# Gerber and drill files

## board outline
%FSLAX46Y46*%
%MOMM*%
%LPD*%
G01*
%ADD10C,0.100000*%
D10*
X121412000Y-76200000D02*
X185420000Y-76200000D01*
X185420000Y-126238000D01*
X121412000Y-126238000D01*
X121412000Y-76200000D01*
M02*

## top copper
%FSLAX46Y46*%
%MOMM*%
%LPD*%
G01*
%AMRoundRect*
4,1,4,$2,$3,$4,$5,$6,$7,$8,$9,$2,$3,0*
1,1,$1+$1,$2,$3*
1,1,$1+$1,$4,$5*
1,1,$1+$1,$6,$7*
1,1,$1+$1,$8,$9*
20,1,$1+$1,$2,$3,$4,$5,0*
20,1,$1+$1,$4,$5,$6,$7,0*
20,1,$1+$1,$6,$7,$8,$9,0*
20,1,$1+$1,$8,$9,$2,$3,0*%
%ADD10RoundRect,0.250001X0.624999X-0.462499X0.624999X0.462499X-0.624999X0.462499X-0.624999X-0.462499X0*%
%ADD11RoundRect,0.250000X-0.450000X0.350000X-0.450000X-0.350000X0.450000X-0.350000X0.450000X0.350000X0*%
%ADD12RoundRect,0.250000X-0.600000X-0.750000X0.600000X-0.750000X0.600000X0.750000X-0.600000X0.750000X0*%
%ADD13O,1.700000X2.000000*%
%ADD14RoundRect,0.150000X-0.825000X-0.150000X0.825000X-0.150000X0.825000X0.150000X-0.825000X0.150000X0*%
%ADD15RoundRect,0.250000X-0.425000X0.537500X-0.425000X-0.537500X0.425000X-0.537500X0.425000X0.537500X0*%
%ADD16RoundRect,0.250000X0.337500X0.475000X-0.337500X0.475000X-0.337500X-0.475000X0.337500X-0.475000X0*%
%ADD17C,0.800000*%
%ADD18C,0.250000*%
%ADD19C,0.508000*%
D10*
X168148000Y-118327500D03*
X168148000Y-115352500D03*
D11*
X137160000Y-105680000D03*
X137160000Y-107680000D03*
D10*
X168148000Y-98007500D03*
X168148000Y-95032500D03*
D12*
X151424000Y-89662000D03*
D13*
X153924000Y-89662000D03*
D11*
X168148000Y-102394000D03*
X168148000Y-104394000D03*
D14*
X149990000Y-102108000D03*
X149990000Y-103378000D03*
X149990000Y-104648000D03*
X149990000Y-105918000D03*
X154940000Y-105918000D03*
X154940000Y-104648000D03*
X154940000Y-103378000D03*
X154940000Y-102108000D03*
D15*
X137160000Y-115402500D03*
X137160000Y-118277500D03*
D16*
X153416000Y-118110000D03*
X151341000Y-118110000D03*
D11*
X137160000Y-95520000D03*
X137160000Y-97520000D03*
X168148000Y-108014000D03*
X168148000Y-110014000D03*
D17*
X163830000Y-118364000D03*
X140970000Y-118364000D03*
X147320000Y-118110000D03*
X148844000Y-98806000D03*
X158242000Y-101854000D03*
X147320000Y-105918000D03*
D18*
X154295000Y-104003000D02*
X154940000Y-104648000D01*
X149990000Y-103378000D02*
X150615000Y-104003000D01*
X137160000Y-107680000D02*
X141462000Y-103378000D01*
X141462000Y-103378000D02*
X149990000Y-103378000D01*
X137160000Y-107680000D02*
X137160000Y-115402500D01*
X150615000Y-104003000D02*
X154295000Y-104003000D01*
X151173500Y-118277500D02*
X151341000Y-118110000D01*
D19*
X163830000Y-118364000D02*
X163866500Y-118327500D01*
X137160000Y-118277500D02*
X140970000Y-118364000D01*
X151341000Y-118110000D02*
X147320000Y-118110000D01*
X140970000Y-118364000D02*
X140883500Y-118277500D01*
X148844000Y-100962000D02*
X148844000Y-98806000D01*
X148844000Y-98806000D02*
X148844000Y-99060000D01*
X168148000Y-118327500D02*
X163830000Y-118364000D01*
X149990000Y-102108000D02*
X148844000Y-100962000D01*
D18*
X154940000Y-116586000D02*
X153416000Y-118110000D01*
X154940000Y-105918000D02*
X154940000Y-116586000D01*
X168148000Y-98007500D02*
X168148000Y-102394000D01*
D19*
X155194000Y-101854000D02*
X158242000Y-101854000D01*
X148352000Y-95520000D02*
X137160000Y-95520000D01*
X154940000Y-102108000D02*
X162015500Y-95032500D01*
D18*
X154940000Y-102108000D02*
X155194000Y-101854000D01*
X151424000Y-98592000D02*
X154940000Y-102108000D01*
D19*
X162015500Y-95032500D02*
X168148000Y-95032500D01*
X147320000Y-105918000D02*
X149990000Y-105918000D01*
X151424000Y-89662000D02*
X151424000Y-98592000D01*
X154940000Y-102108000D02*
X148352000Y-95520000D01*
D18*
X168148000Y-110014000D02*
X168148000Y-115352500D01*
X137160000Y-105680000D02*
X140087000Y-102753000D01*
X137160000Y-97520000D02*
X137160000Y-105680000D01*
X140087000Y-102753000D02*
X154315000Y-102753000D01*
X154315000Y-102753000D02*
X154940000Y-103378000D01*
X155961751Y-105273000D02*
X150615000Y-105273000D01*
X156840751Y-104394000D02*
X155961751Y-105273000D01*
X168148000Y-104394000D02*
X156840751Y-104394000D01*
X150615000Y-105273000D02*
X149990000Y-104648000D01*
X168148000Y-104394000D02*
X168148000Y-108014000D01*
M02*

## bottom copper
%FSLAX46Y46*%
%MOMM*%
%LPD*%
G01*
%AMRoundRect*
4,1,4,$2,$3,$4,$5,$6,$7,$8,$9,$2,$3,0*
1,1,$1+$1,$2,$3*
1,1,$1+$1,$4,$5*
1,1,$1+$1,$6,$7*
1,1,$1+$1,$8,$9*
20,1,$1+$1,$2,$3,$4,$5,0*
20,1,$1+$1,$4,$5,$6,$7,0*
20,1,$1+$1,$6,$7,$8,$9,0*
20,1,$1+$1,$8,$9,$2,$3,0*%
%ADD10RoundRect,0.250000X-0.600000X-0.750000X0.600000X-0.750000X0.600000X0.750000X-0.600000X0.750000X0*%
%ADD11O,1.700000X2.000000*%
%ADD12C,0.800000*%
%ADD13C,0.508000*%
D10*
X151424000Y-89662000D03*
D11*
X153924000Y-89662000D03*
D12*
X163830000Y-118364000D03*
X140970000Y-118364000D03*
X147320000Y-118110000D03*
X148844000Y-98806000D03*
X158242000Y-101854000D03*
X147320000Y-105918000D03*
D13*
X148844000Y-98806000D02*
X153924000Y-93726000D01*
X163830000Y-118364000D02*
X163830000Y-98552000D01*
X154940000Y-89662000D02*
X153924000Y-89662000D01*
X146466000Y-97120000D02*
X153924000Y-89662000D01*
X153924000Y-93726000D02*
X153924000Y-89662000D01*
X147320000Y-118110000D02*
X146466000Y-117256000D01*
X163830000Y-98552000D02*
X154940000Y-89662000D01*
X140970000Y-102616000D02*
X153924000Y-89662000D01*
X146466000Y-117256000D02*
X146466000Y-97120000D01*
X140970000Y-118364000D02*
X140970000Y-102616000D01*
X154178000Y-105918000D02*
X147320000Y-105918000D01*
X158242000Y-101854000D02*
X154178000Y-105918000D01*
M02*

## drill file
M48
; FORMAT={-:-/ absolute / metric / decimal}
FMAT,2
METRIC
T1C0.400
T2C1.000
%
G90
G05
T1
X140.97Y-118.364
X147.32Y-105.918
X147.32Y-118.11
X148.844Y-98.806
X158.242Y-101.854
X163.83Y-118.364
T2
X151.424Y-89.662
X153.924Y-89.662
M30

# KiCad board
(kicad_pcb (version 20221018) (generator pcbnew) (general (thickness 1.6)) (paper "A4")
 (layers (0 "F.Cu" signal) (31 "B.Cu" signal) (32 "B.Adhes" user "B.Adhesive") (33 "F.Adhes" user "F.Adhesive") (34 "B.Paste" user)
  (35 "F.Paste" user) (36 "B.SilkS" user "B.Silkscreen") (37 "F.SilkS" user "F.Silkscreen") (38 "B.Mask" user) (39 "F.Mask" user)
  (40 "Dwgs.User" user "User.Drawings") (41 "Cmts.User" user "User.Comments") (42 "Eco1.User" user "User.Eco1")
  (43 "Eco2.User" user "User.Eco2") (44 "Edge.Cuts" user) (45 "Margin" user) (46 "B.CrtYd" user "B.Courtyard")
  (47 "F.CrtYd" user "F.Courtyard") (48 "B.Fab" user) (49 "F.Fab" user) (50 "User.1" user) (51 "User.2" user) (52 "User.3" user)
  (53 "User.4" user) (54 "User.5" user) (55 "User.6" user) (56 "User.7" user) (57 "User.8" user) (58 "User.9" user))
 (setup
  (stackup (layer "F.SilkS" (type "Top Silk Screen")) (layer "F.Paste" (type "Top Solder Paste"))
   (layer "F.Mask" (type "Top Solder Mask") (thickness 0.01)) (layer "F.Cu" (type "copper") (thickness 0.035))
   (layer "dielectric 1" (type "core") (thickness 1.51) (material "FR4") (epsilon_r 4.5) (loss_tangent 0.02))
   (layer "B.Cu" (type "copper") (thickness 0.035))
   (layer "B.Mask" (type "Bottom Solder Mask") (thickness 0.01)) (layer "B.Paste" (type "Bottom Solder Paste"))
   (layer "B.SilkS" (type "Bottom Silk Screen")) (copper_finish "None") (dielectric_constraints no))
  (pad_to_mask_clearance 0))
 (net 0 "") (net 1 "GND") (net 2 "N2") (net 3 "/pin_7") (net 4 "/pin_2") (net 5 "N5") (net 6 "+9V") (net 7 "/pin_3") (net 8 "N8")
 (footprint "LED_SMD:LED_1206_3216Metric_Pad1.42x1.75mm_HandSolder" (layer "F.Cu") (at 168.148 116.84 90)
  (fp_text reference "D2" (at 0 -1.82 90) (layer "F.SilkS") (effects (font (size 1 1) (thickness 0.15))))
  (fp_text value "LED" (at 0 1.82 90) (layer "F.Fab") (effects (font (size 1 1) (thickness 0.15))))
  (pad "1" smd roundrect (at -1.4875 0 90) (size 1.425 1.75) (layers "F.Cu" "F.Paste" "F.Mask") (roundrect_rratio 0.175439) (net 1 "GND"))
  (pad "2" smd roundrect (at 1.4875 0 90) (size 1.425 1.75) (layers "F.Cu" "F.Paste" "F.Mask") (roundrect_rratio 0.175439) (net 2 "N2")))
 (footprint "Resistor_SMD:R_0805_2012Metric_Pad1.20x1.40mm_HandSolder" (layer "F.Cu") (at 137.16 106.68 -90)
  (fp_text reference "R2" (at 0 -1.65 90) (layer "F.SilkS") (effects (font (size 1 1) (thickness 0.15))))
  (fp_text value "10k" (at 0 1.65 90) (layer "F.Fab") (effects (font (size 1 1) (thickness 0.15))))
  (pad "1" smd roundrect (at -1 0 270) (size 1.2 1.4) (layers "F.Cu" "F.Paste" "F.Mask") (roundrect_rratio 0.208333) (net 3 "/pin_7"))
  (pad "2" smd roundrect (at 1 0 270) (size 1.2 1.4) (layers "F.Cu" "F.Paste" "F.Mask") (roundrect_rratio 0.208333) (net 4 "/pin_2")))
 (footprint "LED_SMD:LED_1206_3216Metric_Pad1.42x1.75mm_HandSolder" (layer "F.Cu") (at 168.148 96.52 90)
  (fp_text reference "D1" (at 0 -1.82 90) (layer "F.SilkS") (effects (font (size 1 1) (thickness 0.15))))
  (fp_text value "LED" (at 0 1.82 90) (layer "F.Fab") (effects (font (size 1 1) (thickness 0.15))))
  (pad "1" smd roundrect (at -1.4875 0 90) (size 1.425 1.75) (layers "F.Cu" "F.Paste" "F.Mask") (roundrect_rratio 0.175439) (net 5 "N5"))
  (pad "2" smd roundrect (at 1.4875 0 90) (size 1.425 1.75) (layers "F.Cu" "F.Paste" "F.Mask") (roundrect_rratio 0.175439) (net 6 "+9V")))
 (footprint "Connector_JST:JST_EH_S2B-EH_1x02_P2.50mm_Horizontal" (layer "F.Cu") (at 151.424 89.662)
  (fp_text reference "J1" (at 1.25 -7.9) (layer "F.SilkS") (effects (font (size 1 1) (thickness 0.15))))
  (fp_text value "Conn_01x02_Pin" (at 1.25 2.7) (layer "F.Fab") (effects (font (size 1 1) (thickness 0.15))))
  (pad "1" thru_hole roundrect (at 0 0) (size 1.7 2) (drill 1) (layers "*.Cu" "*.Mask") (roundrect_rratio 0.147059) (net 6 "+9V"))
  (pad "2" thru_hole oval (at 2.5 0) (size 1.7 2) (drill 1) (layers "*.Cu" "*.Mask") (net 1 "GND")))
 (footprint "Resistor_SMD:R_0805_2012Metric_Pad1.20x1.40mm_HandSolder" (layer "F.Cu") (at 168.148 103.394 -90)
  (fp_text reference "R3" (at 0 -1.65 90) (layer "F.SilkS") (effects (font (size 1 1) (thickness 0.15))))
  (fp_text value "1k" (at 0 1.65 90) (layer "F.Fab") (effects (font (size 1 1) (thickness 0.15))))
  (pad "1" smd roundrect (at -1 0 270) (size 1.2 1.4) (layers "F.Cu" "F.Paste" "F.Mask") (roundrect_rratio 0.208333) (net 5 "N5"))
  (pad "2" smd roundrect (at 1 0 270) (size 1.2 1.4) (layers "F.Cu" "F.Paste" "F.Mask") (roundrect_rratio 0.208333) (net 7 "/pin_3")))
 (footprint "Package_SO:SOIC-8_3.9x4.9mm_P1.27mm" (layer "F.Cu") (at 152.465 104.013)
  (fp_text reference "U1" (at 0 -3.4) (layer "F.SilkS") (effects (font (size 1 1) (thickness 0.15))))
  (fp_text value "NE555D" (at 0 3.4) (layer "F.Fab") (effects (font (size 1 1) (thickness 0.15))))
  (pad "1" smd roundrect (at -2.475 -1.905) (size 1.95 0.6) (layers "F.Cu" "F.Paste" "F.Mask") (roundrect_rratio 0.25) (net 1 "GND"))
  (pad "2" smd roundrect (at -2.475 -0.635) (size 1.95 0.6) (layers "F.Cu" "F.Paste" "F.Mask") (roundrect_rratio 0.25) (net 4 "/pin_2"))
  (pad "3" smd roundrect (at -2.475 0.635) (size 1.95 0.6) (layers "F.Cu" "F.Paste" "F.Mask") (roundrect_rratio 0.25) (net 7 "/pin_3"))
  (pad "4" smd roundrect (at -2.475 1.905) (size 1.95 0.6) (layers "F.Cu" "F.Paste" "F.Mask") (roundrect_rratio 0.25) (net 6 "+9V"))
  (pad "5" smd roundrect (at 2.475 1.905) (size 1.95 0.6) (layers "F.Cu" "F.Paste" "F.Mask") (roundrect_rratio 0.25) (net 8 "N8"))
  (pad "6" smd roundrect (at 2.475 0.635) (size 1.95 0.6) (layers "F.Cu" "F.Paste" "F.Mask") (roundrect_rratio 0.25) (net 4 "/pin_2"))
  (pad "7" smd roundrect (at 2.475 -0.635) (size 1.95 0.6) (layers "F.Cu" "F.Paste" "F.Mask") (roundrect_rratio 0.25) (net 3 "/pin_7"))
  (pad "8" smd roundrect (at 2.475 -1.905) (size 1.95 0.6) (layers "F.Cu" "F.Paste" "F.Mask") (roundrect_rratio 0.25) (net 6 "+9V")))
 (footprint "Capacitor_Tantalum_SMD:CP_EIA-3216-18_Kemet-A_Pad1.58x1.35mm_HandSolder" (layer "F.Cu") (at 137.16 116.84 -90)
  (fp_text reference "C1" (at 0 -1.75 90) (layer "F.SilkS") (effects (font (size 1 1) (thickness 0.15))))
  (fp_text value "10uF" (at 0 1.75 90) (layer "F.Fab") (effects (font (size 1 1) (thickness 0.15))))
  (pad "1" smd roundrect (at -1.4375 0 270) (size 1.575 1.35) (layers "F.Cu" "F.Paste" "F.Mask") (roundrect_rratio 0.185185)
   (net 4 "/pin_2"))
  (pad "2" smd roundrect (at 1.4375 0 270) (size 1.575 1.35) (layers "F.Cu" "F.Paste" "F.Mask") (roundrect_rratio 0.185185) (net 1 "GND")))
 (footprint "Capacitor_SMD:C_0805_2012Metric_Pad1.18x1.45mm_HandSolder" (layer "F.Cu") (at 152.3785 118.11 180)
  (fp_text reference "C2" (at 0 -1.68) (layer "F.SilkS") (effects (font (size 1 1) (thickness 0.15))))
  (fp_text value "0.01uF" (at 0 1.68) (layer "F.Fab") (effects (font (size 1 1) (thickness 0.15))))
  (pad "1" smd roundrect (at -1.0375 0 180) (size 1.175 1.45) (layers "F.Cu" "F.Paste" "F.Mask") (roundrect_rratio 0.212766) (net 8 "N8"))
  (pad "2" smd roundrect (at 1.0375 0 180) (size 1.175 1.45) (layers "F.Cu" "F.Paste" "F.Mask") (roundrect_rratio 0.212766) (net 1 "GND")))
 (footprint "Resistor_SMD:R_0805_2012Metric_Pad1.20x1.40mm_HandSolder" (layer "F.Cu") (at 137.16 96.52 -90)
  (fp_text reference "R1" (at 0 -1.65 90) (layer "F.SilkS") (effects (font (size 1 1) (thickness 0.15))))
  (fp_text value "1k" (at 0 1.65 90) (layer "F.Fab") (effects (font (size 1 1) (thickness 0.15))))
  (pad "1" smd roundrect (at -1 0 270) (size 1.2 1.4) (layers "F.Cu" "F.Paste" "F.Mask") (roundrect_rratio 0.208333) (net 6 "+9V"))
  (pad "2" smd roundrect (at 1 0 270) (size 1.2 1.4) (layers "F.Cu" "F.Paste" "F.Mask") (roundrect_rratio 0.208333) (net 3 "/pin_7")))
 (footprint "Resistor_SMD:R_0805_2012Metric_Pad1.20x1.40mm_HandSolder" (layer "F.Cu") (at 168.148 109.014 -90)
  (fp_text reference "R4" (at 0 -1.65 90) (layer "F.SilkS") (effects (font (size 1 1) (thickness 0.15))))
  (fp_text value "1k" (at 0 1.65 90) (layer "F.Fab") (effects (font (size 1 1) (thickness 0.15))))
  (pad "1" smd roundrect (at -1 0 270) (size 1.2 1.4) (layers "F.Cu" "F.Paste" "F.Mask") (roundrect_rratio 0.208333) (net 7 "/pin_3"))
  (pad "2" smd roundrect (at 1 0 270) (size 1.2 1.4) (layers "F.Cu" "F.Paste" "F.Mask") (roundrect_rratio 0.208333) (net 2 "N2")))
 (gr_rect (start 121.412 76.2) (end 185.42 126.238) (stroke (width 0.1) (type default)) (fill none) (layer "Edge.Cuts"))
 (segment (start 154.295 104.003) (end 154.94 104.648) (width 0.25) (layer "F.Cu") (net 4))
 (segment (start 149.99 103.378) (end 150.615 104.003) (width 0.25) (layer "F.Cu") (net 4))
 (segment (start 137.16 107.68) (end 141.462 103.378) (width 0.25) (layer "F.Cu") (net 4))
 (segment (start 141.462 103.378) (end 149.99 103.378) (width 0.25) (layer "F.Cu") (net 4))
 (segment (start 137.16 107.68) (end 137.16 115.4025) (width 0.25) (layer "F.Cu") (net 4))
 (segment (start 150.615 104.003) (end 154.295 104.003) (width 0.25) (layer "F.Cu") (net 4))
 (segment (start 151.1735 118.2775) (end 151.341 118.11) (width 0.25) (layer "F.Cu") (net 1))
 (segment (start 163.83 118.364) (end 163.8665 118.3275) (width 0.508) (layer "F.Cu") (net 1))
 (segment (start 137.16 118.2775) (end 140.97 118.364) (width 0.508) (layer "F.Cu") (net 1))
 (segment (start 151.341 118.11) (end 147.32 118.11) (width 0.508) (layer "F.Cu") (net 1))
 (segment (start 140.97 118.364) (end 140.8835 118.2775) (width 0.508) (layer "F.Cu") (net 1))
 (segment (start 148.844 100.962) (end 148.844 98.806) (width 0.508) (layer "F.Cu") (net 1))
 (segment (start 148.844 98.806) (end 148.844 99.06) (width 0.508) (layer "F.Cu") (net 1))
 (segment (start 168.148 118.3275) (end 163.83 118.364) (width 0.508) (layer "F.Cu") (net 1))
 (segment (start 149.99 102.108) (end 148.844 100.962) (width 0.508) (layer "F.Cu") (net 1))
 (via (at 163.83 118.364) (size 0.8) (drill 0.4) (layers "F.Cu" "B.Cu") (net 1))
 (via (at 140.97 118.364) (size 0.8) (drill 0.4) (layers "F.Cu" "B.Cu") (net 1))
 (via (at 147.32 118.11) (size 0.8) (drill 0.4) (layers "F.Cu" "B.Cu") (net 1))
 (via (at 148.844 98.806) (size 0.8) (drill 0.4) (layers "F.Cu" "B.Cu") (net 1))
 (segment (start 148.844 98.806) (end 153.924 93.726) (width 0.508) (layer "B.Cu") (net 1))
 (segment (start 163.83 118.364) (end 163.83 98.552) (width 0.508) (layer "B.Cu") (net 1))
 (segment (start 154.94 89.662) (end 153.924 89.662) (width 0.508) (layer "B.Cu") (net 1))
 (segment (start 146.466 97.12) (end 153.924 89.662) (width 0.508) (layer "B.Cu") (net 1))
 (segment (start 153.924 93.726) (end 153.924 89.662) (width 0.508) (layer "B.Cu") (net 1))
 (segment (start 147.32 118.11) (end 146.466 117.256) (width 0.508) (layer "B.Cu") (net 1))
 (segment (start 163.83 98.552) (end 154.94 89.662) (width 0.508) (layer "B.Cu") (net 1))
 (segment (start 140.97 102.616) (end 153.924 89.662) (width 0.508) (layer "B.Cu") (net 1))
 (segment (start 146.466 117.256) (end 146.466 97.12) (width 0.508) (layer "B.Cu") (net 1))
 (segment (start 140.97 118.364) (end 140.97 102.616) (width 0.508) (layer "B.Cu") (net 1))
 (segment (start 154.94 116.586) (end 153.416 118.11) (width 0.25) (layer "F.Cu") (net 8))
 (segment (start 154.94 105.918) (end 154.94 116.586) (width 0.25) (layer "F.Cu") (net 8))
 (segment (start 168.148 98.0075) (end 168.148 102.394) (width 0.25) (layer "F.Cu") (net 5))
 (segment (start 155.194 101.854) (end 158.242 101.854) (width 0.508) (layer "F.Cu") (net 6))
 (segment (start 148.352 95.52) (end 137.16 95.52) (width 0.508) (layer "F.Cu") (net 6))
 (segment (start 154.94 102.108) (end 162.0155 95.0325) (width 0.508) (layer "F.Cu") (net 6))
 (segment (start 154.94 102.108) (end 155.194 101.854) (width 0.25) (layer "F.Cu") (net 6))
 (segment (start 151.424 98.592) (end 154.94 102.108) (width 0.25) (layer "F.Cu") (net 6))
 (segment (start 162.0155 95.0325) (end 168.148 95.0325) (width 0.508) (layer "F.Cu") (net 6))
 (segment (start 147.32 105.918) (end 149.99 105.918) (width 0.508) (layer "F.Cu") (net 6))
 (segment (start 151.424 89.662) (end 151.424 98.592) (width 0.508) (layer "F.Cu") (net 6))
 (segment (start 154.94 102.108) (end 148.352 95.52) (width 0.508) (layer "F.Cu") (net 6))
 (via (at 158.242 101.854) (size 0.8) (drill 0.4) (layers "F.Cu" "B.Cu") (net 6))
 (via (at 147.32 105.918) (size 0.8) (drill 0.4) (layers "F.Cu" "B.Cu") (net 6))
 (segment (start 154.178 105.918) (end 147.32 105.918) (width 0.508) (layer "B.Cu") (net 6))
 (segment (start 158.242 101.854) (end 154.178 105.918) (width 0.508) (layer "B.Cu") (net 6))
 (segment (start 168.148 110.014) (end 168.148 115.3525) (width 0.25) (layer "F.Cu") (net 2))
 (segment (start 137.16 105.68) (end 140.087 102.753) (width 0.25) (layer "F.Cu") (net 3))
 (segment (start 137.16 97.52) (end 137.16 105.68) (width 0.25) (layer "F.Cu") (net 3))
 (segment (start 140.087 102.753) (end 154.315 102.753) (width 0.25) (layer "F.Cu") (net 3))
 (segment (start 154.315 102.753) (end 154.94 103.378) (width 0.25) (layer "F.Cu") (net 3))
 (segment (start 155.961751 105.273) (end 150.615 105.273) (width 0.25) (layer "F.Cu") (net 7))
 (segment (start 156.840751 104.394) (end 155.961751 105.273) (width 0.25) (layer "F.Cu") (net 7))
 (segment (start 168.148 104.394) (end 156.840751 104.394) (width 0.25) (layer "F.Cu") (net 7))
 (segment (start 150.615 105.273) (end 149.99 104.648) (width 0.25) (layer "F.Cu") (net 7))
 (segment (start 168.148 104.394) (end 168.148 108.014) (width 0.25) (layer "F.Cu") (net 7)))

